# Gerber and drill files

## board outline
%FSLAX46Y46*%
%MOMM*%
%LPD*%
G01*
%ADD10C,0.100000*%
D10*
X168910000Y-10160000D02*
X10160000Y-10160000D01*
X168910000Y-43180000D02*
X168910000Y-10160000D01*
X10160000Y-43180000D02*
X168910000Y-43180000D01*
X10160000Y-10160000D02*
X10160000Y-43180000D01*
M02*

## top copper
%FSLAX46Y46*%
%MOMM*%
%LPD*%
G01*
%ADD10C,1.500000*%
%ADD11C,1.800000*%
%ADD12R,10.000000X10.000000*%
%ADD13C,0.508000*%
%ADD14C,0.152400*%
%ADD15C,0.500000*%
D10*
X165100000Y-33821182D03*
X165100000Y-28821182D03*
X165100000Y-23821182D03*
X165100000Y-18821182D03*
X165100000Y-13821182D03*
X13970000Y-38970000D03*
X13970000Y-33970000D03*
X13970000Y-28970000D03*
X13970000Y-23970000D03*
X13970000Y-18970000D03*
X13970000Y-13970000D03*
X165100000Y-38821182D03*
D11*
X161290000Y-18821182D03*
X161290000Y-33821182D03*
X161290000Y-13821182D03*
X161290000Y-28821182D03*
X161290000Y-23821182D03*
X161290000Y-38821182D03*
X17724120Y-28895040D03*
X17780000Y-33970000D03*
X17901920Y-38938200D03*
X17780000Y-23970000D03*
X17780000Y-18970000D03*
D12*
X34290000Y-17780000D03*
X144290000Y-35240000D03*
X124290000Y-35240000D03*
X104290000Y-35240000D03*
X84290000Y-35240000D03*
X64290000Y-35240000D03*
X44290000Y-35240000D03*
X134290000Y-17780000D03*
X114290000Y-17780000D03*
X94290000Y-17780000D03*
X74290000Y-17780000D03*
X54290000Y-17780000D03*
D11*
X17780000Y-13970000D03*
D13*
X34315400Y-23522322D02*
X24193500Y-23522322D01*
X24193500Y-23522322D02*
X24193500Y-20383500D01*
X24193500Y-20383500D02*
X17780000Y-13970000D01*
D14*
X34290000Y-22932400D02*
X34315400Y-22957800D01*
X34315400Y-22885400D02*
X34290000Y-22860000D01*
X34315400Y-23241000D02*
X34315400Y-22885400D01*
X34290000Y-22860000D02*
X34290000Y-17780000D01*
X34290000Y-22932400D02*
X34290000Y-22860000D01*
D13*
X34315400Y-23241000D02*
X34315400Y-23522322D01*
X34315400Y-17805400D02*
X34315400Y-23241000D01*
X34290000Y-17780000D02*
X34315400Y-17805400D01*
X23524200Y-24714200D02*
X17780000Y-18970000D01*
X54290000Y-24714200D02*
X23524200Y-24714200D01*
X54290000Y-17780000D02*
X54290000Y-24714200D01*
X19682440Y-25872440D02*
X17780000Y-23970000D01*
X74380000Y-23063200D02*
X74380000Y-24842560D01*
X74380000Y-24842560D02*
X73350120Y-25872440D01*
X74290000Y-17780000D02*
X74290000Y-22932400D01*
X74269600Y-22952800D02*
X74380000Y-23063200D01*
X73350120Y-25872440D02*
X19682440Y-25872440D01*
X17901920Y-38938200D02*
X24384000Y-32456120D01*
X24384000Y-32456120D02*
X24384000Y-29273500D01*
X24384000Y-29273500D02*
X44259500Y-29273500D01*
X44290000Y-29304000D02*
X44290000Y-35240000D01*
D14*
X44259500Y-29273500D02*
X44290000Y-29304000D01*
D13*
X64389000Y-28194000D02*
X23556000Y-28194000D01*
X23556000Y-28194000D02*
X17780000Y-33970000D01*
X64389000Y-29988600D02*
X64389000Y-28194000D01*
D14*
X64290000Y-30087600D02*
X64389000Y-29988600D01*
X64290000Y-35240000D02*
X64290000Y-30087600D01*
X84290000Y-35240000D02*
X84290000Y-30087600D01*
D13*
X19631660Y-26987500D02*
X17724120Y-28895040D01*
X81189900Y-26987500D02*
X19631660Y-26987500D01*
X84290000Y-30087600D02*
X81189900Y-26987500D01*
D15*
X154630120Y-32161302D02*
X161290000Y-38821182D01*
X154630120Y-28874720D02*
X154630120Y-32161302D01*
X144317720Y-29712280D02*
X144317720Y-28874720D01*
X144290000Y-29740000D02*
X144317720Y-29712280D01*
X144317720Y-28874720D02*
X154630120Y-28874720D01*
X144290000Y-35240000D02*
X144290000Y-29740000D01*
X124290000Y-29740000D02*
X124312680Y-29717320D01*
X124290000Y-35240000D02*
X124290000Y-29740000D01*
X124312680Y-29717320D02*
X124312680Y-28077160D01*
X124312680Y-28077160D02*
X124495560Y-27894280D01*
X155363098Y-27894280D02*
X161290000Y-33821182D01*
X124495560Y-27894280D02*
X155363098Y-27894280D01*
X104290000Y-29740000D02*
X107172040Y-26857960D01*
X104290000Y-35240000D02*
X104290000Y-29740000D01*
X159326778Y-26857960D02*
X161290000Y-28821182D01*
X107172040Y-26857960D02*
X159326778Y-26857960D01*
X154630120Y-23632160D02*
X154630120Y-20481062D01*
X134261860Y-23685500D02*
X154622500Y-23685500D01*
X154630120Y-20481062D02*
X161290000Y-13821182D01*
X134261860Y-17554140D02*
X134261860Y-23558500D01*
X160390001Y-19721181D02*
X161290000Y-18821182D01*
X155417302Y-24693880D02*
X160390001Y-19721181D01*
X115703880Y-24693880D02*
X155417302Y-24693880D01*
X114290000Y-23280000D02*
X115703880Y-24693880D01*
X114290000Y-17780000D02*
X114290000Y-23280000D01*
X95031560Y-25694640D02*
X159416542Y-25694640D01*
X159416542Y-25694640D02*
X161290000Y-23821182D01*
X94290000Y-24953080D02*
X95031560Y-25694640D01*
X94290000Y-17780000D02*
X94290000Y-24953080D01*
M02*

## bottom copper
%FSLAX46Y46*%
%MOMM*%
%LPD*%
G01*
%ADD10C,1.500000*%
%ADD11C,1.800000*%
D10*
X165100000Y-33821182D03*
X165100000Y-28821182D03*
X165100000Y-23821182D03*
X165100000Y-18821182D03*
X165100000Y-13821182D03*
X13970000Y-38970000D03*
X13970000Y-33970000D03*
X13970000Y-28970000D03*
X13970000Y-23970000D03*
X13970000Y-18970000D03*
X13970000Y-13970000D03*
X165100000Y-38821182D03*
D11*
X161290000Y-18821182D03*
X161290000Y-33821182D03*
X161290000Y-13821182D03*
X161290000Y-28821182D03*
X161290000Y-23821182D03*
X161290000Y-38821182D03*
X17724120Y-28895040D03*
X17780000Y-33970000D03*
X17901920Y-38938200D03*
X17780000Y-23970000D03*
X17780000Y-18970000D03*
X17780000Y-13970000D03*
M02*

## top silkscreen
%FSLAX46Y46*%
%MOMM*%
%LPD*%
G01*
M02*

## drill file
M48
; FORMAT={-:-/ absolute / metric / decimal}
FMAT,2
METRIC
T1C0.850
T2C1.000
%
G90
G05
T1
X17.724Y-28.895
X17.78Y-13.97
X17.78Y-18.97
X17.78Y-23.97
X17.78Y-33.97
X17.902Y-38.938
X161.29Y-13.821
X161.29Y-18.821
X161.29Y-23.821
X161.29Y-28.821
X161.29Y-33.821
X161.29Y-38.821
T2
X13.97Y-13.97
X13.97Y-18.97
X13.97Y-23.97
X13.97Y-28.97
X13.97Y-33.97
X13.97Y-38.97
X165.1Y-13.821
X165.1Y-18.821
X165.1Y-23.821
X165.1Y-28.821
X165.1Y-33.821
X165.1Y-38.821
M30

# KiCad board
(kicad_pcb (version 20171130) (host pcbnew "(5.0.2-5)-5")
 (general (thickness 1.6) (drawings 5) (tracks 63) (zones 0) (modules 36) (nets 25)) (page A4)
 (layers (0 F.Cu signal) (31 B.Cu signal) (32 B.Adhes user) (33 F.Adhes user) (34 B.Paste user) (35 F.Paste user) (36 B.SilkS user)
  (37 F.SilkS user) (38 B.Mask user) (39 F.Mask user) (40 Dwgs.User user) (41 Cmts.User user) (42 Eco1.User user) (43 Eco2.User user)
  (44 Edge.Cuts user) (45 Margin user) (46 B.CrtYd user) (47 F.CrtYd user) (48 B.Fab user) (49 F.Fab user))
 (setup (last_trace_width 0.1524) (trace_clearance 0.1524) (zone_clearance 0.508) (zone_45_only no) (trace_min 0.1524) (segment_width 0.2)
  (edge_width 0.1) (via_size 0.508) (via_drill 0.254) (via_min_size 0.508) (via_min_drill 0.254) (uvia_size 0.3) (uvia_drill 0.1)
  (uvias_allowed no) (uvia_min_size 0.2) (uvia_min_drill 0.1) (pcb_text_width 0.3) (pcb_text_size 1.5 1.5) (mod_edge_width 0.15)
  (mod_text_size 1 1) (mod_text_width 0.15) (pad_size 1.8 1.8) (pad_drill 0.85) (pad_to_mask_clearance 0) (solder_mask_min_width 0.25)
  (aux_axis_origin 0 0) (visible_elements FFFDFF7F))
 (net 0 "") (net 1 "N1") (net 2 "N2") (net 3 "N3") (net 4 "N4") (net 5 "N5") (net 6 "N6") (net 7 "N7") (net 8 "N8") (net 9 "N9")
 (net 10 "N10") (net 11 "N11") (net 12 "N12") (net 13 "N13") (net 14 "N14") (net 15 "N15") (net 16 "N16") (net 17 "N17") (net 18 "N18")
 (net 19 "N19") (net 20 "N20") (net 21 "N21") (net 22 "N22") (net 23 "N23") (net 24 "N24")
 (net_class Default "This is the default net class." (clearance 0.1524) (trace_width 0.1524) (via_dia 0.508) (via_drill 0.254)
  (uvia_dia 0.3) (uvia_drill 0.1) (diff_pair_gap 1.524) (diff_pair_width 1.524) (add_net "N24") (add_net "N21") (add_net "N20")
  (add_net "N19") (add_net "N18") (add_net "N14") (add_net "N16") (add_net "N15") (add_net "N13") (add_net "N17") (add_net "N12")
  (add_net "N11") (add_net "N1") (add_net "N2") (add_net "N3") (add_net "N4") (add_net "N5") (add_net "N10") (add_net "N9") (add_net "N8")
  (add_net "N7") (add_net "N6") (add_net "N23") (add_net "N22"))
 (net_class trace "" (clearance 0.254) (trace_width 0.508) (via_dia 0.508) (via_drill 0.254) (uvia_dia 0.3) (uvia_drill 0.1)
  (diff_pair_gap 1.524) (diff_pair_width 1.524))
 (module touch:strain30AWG (layer B.Cu) (at 165.1 33.821182)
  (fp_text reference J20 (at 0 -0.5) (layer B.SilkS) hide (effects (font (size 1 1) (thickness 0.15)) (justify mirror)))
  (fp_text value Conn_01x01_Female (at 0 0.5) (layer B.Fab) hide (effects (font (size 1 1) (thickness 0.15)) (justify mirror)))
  (pad 1 thru_hole circle (at 0 0) (size 1.5 1.5) (drill 1) (layers *.Cu) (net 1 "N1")))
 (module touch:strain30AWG (layer B.Cu) (at 165.1 28.821182)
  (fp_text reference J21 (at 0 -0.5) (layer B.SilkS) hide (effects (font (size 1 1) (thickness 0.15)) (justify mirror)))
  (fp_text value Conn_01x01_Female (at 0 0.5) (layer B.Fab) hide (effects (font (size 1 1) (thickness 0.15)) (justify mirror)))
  (pad 1 thru_hole circle (at 0 0) (size 1.5 1.5) (drill 1) (layers *.Cu) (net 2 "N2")))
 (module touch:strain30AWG (layer B.Cu) (at 165.1 23.821182)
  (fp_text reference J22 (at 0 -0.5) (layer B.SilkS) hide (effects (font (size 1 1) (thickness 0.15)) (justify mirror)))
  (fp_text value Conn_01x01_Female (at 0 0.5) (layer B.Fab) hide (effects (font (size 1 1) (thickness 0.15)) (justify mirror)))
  (pad 1 thru_hole circle (at 0 0) (size 1.5 1.5) (drill 1) (layers *.Cu) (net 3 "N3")))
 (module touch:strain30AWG (layer B.Cu) (at 165.1 18.821182)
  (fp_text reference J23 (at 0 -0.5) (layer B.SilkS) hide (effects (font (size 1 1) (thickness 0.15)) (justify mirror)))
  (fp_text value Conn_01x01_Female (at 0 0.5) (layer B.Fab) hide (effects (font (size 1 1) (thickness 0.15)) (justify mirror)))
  (pad 1 thru_hole circle (at 0 0) (size 1.5 1.5) (drill 1) (layers *.Cu) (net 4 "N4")))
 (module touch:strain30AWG (layer B.Cu) (at 165.1 13.821182)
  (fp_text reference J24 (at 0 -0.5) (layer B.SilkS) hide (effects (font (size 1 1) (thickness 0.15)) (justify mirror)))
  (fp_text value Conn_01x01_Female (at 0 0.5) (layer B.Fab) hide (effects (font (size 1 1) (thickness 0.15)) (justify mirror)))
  (pad 1 thru_hole circle (at 0 0) (size 1.5 1.5) (drill 1) (layers *.Cu) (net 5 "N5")))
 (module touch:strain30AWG (layer F.Cu) (at 13.97 38.97)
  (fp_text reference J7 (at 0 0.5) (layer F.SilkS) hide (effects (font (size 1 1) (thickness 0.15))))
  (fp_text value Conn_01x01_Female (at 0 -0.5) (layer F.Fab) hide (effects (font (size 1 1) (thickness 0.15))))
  (pad 1 thru_hole circle (at 0 0) (size 1.5 1.5) (drill 1) (layers *.Cu) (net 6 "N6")))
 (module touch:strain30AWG (layer F.Cu) (at 13.97 33.97)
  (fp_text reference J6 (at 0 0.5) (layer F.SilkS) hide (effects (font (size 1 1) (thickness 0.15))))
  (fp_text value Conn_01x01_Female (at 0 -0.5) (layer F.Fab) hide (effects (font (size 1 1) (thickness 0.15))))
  (pad 1 thru_hole circle (at 0 0) (size 1.5 1.5) (drill 1) (layers *.Cu) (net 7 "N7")))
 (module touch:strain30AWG (layer F.Cu) (at 13.97 28.97)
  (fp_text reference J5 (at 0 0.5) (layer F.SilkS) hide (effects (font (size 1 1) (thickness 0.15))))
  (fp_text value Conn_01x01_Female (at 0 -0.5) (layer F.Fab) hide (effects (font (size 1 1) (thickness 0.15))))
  (pad 1 thru_hole circle (at 0 0) (size 1.5 1.5) (drill 1) (layers *.Cu) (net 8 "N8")))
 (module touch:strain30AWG (layer F.Cu) (at 13.97 23.97)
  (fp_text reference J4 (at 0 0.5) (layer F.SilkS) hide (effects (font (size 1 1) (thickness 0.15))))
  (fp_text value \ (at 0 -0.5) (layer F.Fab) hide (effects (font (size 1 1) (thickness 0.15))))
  (pad 1 thru_hole circle (at 0 0) (size 1.5 1.5) (drill 1) (layers *.Cu) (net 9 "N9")))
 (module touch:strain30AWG (layer F.Cu) (at 13.97 18.97)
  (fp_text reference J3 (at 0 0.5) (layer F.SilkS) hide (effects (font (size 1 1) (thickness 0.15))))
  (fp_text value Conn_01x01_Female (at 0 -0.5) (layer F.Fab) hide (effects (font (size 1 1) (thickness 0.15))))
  (pad 1 thru_hole circle (at 0 0) (size 1.5 1.5) (drill 1) (layers *.Cu) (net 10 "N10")))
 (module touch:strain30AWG (layer F.Cu) (at 13.97 13.97)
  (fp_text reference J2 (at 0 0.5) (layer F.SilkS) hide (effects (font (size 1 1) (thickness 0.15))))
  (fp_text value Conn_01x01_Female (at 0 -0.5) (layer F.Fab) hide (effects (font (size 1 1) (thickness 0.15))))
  (pad 1 thru_hole circle (at 0 0) (size 1.5 1.5) (drill 1) (layers *.Cu) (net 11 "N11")))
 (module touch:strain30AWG (layer B.Cu) (at 165.1 38.821182)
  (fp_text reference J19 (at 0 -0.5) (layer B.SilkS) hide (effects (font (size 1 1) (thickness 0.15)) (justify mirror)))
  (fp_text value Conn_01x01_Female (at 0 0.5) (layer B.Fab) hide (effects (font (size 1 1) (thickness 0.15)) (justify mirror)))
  (pad 1 thru_hole circle (at 0 0) (size 1.5 1.5) (drill 1) (layers *.Cu) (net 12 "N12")))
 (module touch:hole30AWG (layer B.Cu) (at 161.29 18.821182)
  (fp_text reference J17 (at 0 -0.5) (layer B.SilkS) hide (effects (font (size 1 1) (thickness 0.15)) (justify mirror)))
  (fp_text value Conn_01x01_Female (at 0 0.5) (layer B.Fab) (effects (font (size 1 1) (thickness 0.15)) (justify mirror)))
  (pad 1 thru_hole circle (at 0 0) (size 1.8 1.8) (drill 0.85) (layers *.Cu *.Mask) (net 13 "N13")))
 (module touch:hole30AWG (layer B.Cu) (at 161.29 33.821182)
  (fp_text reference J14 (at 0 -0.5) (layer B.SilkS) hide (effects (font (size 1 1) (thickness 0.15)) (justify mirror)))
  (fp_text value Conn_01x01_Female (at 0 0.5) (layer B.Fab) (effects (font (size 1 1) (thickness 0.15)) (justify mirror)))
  (pad 1 thru_hole circle (at 0 0) (size 1.8 1.8) (drill 0.85) (layers *.Cu *.Mask) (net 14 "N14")))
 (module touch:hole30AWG (layer B.Cu) (at 161.29 13.821182)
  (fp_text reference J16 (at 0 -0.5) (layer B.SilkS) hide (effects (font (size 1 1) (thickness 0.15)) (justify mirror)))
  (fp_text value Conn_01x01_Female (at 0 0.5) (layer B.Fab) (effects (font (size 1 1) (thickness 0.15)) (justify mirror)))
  (pad 1 thru_hole circle (at 0 0) (size 1.8 1.8) (drill 0.85) (layers *.Cu *.Mask) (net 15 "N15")))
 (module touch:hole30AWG (layer B.Cu) (at 161.29 28.821182)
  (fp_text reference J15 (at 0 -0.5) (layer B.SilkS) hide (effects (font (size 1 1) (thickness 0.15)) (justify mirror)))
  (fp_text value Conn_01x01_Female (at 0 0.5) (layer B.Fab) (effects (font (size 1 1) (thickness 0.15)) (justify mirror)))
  (pad 1 thru_hole circle (at 0 0) (size 1.8 1.8) (drill 0.85) (layers *.Cu *.Mask) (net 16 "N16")))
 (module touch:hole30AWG (layer B.Cu) (at 161.29 23.821182)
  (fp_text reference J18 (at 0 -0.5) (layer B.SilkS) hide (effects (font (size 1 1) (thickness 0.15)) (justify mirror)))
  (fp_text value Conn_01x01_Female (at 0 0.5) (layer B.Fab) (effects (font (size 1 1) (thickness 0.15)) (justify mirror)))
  (pad 1 thru_hole circle (at 0 0) (size 1.8 1.8) (drill 0.85) (layers *.Cu *.Mask) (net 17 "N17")))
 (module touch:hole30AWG (layer B.Cu) (at 161.29 38.821182)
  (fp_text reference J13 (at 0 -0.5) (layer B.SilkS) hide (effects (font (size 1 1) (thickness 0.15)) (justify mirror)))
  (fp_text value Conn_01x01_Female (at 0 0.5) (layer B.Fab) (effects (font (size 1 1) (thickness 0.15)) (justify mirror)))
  (pad 1 thru_hole circle (at 0 0) (size 1.8 1.8) (drill 0.85) (layers *.Cu *.Mask) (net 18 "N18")))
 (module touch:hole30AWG (layer F.Cu) (at 17.72412 28.89504)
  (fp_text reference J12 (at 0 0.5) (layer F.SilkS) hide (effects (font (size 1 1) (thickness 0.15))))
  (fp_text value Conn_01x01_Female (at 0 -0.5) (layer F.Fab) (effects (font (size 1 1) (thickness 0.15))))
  (pad 1 thru_hole circle (at 0 0) (size 1.8 1.8) (drill 0.85) (layers *.Cu *.Mask) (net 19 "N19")))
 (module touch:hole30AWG (layer F.Cu) (at 17.78 33.97)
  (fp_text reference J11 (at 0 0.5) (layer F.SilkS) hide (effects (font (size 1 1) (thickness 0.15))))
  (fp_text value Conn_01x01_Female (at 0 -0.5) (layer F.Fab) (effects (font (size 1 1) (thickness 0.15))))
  (pad 1 thru_hole circle (at 0 0) (size 1.8 1.8) (drill 0.85) (layers *.Cu *.Mask) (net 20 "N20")))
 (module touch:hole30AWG (layer F.Cu) (at 17.90192 38.9382)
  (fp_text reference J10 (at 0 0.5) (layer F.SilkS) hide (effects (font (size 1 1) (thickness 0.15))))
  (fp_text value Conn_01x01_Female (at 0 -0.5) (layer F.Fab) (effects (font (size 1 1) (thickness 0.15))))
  (pad 1 thru_hole circle (at 0 0) (size 1.8 1.8) (drill 0.85) (layers *.Cu *.Mask) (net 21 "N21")))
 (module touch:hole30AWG (layer F.Cu) (at 17.78 23.97)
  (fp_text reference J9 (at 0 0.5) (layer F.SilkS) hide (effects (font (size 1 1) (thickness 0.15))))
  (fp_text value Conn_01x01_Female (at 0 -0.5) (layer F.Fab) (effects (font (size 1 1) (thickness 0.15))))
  (pad 1 thru_hole circle (at 0 0) (size 1.8 1.8) (drill 0.85) (layers *.Cu *.Mask) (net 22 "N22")))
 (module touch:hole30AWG (layer F.Cu) (at 17.78 18.97)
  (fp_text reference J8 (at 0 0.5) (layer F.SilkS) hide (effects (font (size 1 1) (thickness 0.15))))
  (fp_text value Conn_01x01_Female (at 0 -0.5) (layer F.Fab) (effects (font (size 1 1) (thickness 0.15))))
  (pad 1 thru_hole circle (at 0 0) (size 1.8 1.8) (drill 0.85) (layers *.Cu *.Mask) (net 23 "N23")))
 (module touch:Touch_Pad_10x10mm (layer F.Cu) (at 34.29 17.78)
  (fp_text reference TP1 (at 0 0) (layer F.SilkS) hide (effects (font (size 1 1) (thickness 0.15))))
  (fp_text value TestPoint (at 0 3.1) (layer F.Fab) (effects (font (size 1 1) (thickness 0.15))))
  (pad 1 smd rect (at 0 0) (size 10 10) (layers F.Cu F.Mask) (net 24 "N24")))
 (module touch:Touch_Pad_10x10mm (layer F.Cu) (at 144.29 35.24)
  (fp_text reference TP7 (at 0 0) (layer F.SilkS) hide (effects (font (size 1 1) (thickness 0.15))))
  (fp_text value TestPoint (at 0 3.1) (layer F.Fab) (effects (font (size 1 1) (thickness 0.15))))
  (pad 1 smd rect (at 0 0) (size 10 10) (layers F.Cu F.Mask) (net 18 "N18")))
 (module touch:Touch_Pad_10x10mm (layer F.Cu) (at 124.29 35.24)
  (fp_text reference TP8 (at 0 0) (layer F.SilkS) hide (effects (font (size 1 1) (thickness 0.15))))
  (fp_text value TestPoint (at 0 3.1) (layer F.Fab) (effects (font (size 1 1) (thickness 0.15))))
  (pad 1 smd rect (at 0 0) (size 10 10) (layers F.Cu F.Mask) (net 14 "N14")))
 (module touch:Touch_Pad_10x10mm (layer F.Cu) (at 104.29 35.24)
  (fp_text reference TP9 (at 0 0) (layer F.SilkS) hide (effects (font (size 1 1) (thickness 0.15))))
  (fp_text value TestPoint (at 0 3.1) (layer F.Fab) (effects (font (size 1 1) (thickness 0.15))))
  (pad 1 smd rect (at 0 0) (size 10 10) (layers F.Cu F.Mask) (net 16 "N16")))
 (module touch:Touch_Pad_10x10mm (layer F.Cu) (at 84.29 35.24)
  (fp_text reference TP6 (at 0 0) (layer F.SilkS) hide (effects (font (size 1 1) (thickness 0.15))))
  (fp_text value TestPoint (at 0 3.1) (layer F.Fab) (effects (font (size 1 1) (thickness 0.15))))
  (pad 1 smd rect (at 0 0) (size 10 10) (layers F.Cu F.Mask) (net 19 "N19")))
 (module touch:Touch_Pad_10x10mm (layer F.Cu) (at 64.29 35.24)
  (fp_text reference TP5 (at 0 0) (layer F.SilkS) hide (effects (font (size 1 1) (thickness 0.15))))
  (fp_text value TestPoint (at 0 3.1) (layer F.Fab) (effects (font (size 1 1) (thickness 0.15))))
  (pad 1 smd rect (at 0 0) (size 10 10) (layers F.Cu F.Mask) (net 20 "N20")))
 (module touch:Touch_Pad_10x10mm (layer F.Cu) (at 44.29 35.24)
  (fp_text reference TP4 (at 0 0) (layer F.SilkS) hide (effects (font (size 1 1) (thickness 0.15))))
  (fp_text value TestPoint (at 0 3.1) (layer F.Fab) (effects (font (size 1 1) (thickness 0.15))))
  (pad 1 smd rect (at 0 0) (size 10 10) (layers F.Cu F.Mask) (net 21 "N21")))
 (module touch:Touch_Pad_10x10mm (layer F.Cu) (at 134.29 17.78)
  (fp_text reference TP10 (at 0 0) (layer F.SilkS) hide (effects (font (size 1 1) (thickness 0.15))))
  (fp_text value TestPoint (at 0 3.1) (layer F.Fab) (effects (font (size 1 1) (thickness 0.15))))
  (pad 1 smd rect (at 0 0) (size 10 10) (layers F.Cu F.Mask) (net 15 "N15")))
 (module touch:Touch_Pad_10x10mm (layer F.Cu) (at 114.29 17.78)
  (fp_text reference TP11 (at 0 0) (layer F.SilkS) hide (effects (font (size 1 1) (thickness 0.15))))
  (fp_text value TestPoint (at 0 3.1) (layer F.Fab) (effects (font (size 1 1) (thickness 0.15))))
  (pad 1 smd rect (at 0 0) (size 10 10) (layers F.Cu F.Mask) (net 13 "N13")))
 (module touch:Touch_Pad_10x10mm (layer F.Cu) (at 94.29 17.78)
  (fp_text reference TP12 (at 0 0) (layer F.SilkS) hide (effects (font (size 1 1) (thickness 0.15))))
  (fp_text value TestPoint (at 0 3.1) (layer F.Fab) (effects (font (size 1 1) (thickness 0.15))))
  (pad 1 smd rect (at 0 0) (size 10 10) (layers F.Cu F.Mask) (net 17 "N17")))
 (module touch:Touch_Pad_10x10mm (layer F.Cu) (at 74.29 17.78)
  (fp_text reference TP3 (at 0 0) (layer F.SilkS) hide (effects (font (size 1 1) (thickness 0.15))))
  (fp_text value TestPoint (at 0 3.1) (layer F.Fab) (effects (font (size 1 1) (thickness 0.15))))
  (pad 1 smd rect (at 0 0) (size 10 10) (layers F.Cu F.Mask) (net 22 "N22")))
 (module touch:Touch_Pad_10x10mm (layer F.Cu) (at 54.29 17.78)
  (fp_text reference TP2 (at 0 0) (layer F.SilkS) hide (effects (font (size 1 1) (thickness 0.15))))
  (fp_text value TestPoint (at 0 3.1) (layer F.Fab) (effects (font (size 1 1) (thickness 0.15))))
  (pad 1 smd rect (at 0 0) (size 10 10) (layers F.Cu F.Mask) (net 23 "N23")))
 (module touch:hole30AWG (layer F.Cu) (at 17.78 13.97)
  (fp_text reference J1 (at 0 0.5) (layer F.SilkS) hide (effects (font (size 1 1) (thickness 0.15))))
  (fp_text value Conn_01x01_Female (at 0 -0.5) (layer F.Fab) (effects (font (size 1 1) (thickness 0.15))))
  (pad 1 thru_hole circle (at 0 0) (size 1.8 1.8) (drill 0.85) (layers *.Cu *.Mask) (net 24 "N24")))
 (gr_line (start 168.91 10.16) (end 10.16 10.16) (layer Edge.Cuts) (width 0.1))
 (gr_line (start 168.91 43.18) (end 168.91 10.16) (layer Edge.Cuts) (width 0.1))
 (gr_line (start 10.16 43.18) (end 168.91 43.18) (layer Edge.Cuts) (width 0.1))
 (gr_line (start 10.16 10.16) (end 10.16 43.18) (layer Edge.Cuts) (width 0.1))
 (segment (start 34.3154 23.522322) (end 24.1935 23.522322) (width 0.508) (layer F.Cu) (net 24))
 (segment (start 24.1935 23.522322) (end 24.1935 20.3835) (width 0.508) (layer F.Cu) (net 24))
 (segment (start 24.1935 20.3835) (end 17.78 13.97) (width 0.508) (layer F.Cu) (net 24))
 (segment (start 34.29 22.9324) (end 34.3154 22.9578) (width 0.1524) (layer F.Cu) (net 24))
 (segment (start 34.3154 22.8854) (end 34.29 22.86) (width 0.1524) (layer F.Cu) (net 24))
 (segment (start 34.3154 23.241) (end 34.3154 22.8854) (width 0.1524) (layer F.Cu) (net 24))
 (segment (start 34.29 22.86) (end 34.29 17.78) (width 0.1524) (layer F.Cu) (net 24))
 (segment (start 34.29 22.9324) (end 34.29 22.86) (width 0.1524) (layer F.Cu) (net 24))
 (segment (start 34.3154 23.241) (end 34.3154 23.522322) (width 0.508) (layer F.Cu) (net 24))
 (segment (start 34.3154 17.8054) (end 34.3154 23.241) (width 0.508) (layer F.Cu) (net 24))
 (segment (start 34.29 17.78) (end 34.3154 17.8054) (width 0.508) (layer F.Cu) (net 24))
 (segment (start 23.5242 24.7142) (end 17.78 18.97) (width 0.508) (layer F.Cu) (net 23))
 (segment (start 54.29 24.7142) (end 23.5242 24.7142) (width 0.508) (layer F.Cu) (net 23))
 (segment (start 54.29 17.78) (end 54.29 24.7142) (width 0.508) (layer F.Cu) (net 23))
 (segment (start 19.68244 25.87244) (end 17.78 23.97) (width 0.508) (layer F.Cu) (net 22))
 (segment (start 74.38 23.0632) (end 74.38 24.84256) (width 0.508) (layer F.Cu) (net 22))
 (segment (start 74.38 24.84256) (end 73.35012 25.87244) (width 0.508) (layer F.Cu) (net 22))
 (segment (start 74.29 17.78) (end 74.29 22.9324) (width 0.508) (layer F.Cu) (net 22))
 (segment (start 74.2696 22.9528) (end 74.38 23.0632) (width 0.508) (layer F.Cu) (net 22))
 (segment (start 73.35012 25.87244) (end 19.68244 25.87244) (width 0.508) (layer F.Cu) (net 22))
 (segment (start 17.90192 38.9382) (end 24.384 32.45612) (width 0.508) (layer F.Cu) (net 21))
 (segment (start 24.384 32.45612) (end 24.384 29.2735) (width 0.508) (layer F.Cu) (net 21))
 (segment (start 24.384 29.2735) (end 44.2595 29.2735) (width 0.508) (layer F.Cu) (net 21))
 (segment (start 44.29 29.304) (end 44.29 35.24) (width 0.508) (layer F.Cu) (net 21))
 (segment (start 44.2595 29.2735) (end 44.29 29.304) (width 0.1524) (layer F.Cu) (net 21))
 (segment (start 64.389 28.194) (end 23.556 28.194) (width 0.508) (layer F.Cu) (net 20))
 (segment (start 23.556 28.194) (end 17.78 33.97) (width 0.508) (layer F.Cu) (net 20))
 (segment (start 64.389 29.9886) (end 64.389 28.194) (width 0.508) (layer F.Cu) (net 20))
 (segment (start 64.29 30.0876) (end 64.389 29.9886) (width 0.1524) (layer F.Cu) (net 20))
 (segment (start 64.29 35.24) (end 64.29 30.0876) (width 0.1524) (layer F.Cu) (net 20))
 (segment (start 84.29 35.24) (end 84.29 30.0876) (width 0.1524) (layer F.Cu) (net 19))
 (segment (start 19.63166 26.9875) (end 17.72412 28.89504) (width 0.508) (layer F.Cu) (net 19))
 (segment (start 81.1899 26.9875) (end 19.63166 26.9875) (width 0.508) (layer F.Cu) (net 19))
 (segment (start 84.29 30.0876) (end 81.1899 26.9875) (width 0.508) (layer F.Cu) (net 19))
 (segment (start 154.63012 32.161302) (end 161.29 38.821182) (width 0.5) (layer F.Cu) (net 18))
 (segment (start 154.63012 28.87472) (end 154.63012 32.161302) (width 0.5) (layer F.Cu) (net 18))
 (segment (start 144.31772 29.71228) (end 144.31772 28.87472) (width 0.5) (layer F.Cu) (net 18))
 (segment (start 144.29 29.74) (end 144.31772 29.71228) (width 0.5) (layer F.Cu) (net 18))
 (segment (start 144.31772 28.87472) (end 154.63012 28.87472) (width 0.5) (layer F.Cu) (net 18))
 (segment (start 144.29 35.24) (end 144.29 29.74) (width 0.5) (layer F.Cu) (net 18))
 (segment (start 124.29 29.74) (end 124.31268 29.71732) (width 0.5) (layer F.Cu) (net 14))
 (segment (start 124.29 35.24) (end 124.29 29.74) (width 0.5) (layer F.Cu) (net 14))
 (segment (start 124.31268 29.71732) (end 124.31268 28.07716) (width 0.5) (layer F.Cu) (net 14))
 (segment (start 124.31268 28.07716) (end 124.49556 27.89428) (width 0.5) (layer F.Cu) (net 14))
 (segment (start 155.363098 27.89428) (end 161.29 33.821182) (width 0.5) (layer F.Cu) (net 14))
 (segment (start 124.49556 27.89428) (end 155.363098 27.89428) (width 0.5) (layer F.Cu) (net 14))
 (segment (start 104.29 29.74) (end 107.17204 26.85796) (width 0.5) (layer F.Cu) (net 16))
 (segment (start 104.29 35.24) (end 104.29 29.74) (width 0.5) (layer F.Cu) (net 16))
 (segment (start 159.326778 26.85796) (end 161.29 28.821182) (width 0.5) (layer F.Cu) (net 16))
 (segment (start 107.17204 26.85796) (end 159.326778 26.85796) (width 0.5) (layer F.Cu) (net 16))
 (segment (start 154.63012 23.63216) (end 154.63012 20.481062) (width 0.5) (layer F.Cu) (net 15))
 (segment (start 134.26186 23.6855) (end 154.6225 23.6855) (width 0.5) (layer F.Cu) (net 15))
 (segment (start 154.63012 20.481062) (end 161.29 13.821182) (width 0.5) (layer F.Cu) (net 15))
 (segment (start 134.26186 17.55414) (end 134.26186 23.5585) (width 0.5) (layer F.Cu) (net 15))
 (segment (start 160.390001 19.721181) (end 161.29 18.821182) (width 0.5) (layer F.Cu) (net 13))
 (segment (start 155.417302 24.69388) (end 160.390001 19.721181) (width 0.5) (layer F.Cu) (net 13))
 (segment (start 115.70388 24.69388) (end 155.417302 24.69388) (width 0.5) (layer F.Cu) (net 13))
 (segment (start 114.29 23.28) (end 115.70388 24.69388) (width 0.5) (layer F.Cu) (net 13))
 (segment (start 114.29 17.78) (end 114.29 23.28) (width 0.5) (layer F.Cu) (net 13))
 (segment (start 95.03156 25.69464) (end 159.416542 25.69464) (width 0.5) (layer F.Cu) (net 17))
 (segment (start 159.416542 25.69464) (end 161.29 23.821182) (width 0.5) (layer F.Cu) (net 17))
 (segment (start 94.29 24.95308) (end 95.03156 25.69464) (width 0.5) (layer F.Cu) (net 17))
 (segment (start 94.29 17.78) (end 94.29 24.95308) (width 0.5) (layer F.Cu) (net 17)))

